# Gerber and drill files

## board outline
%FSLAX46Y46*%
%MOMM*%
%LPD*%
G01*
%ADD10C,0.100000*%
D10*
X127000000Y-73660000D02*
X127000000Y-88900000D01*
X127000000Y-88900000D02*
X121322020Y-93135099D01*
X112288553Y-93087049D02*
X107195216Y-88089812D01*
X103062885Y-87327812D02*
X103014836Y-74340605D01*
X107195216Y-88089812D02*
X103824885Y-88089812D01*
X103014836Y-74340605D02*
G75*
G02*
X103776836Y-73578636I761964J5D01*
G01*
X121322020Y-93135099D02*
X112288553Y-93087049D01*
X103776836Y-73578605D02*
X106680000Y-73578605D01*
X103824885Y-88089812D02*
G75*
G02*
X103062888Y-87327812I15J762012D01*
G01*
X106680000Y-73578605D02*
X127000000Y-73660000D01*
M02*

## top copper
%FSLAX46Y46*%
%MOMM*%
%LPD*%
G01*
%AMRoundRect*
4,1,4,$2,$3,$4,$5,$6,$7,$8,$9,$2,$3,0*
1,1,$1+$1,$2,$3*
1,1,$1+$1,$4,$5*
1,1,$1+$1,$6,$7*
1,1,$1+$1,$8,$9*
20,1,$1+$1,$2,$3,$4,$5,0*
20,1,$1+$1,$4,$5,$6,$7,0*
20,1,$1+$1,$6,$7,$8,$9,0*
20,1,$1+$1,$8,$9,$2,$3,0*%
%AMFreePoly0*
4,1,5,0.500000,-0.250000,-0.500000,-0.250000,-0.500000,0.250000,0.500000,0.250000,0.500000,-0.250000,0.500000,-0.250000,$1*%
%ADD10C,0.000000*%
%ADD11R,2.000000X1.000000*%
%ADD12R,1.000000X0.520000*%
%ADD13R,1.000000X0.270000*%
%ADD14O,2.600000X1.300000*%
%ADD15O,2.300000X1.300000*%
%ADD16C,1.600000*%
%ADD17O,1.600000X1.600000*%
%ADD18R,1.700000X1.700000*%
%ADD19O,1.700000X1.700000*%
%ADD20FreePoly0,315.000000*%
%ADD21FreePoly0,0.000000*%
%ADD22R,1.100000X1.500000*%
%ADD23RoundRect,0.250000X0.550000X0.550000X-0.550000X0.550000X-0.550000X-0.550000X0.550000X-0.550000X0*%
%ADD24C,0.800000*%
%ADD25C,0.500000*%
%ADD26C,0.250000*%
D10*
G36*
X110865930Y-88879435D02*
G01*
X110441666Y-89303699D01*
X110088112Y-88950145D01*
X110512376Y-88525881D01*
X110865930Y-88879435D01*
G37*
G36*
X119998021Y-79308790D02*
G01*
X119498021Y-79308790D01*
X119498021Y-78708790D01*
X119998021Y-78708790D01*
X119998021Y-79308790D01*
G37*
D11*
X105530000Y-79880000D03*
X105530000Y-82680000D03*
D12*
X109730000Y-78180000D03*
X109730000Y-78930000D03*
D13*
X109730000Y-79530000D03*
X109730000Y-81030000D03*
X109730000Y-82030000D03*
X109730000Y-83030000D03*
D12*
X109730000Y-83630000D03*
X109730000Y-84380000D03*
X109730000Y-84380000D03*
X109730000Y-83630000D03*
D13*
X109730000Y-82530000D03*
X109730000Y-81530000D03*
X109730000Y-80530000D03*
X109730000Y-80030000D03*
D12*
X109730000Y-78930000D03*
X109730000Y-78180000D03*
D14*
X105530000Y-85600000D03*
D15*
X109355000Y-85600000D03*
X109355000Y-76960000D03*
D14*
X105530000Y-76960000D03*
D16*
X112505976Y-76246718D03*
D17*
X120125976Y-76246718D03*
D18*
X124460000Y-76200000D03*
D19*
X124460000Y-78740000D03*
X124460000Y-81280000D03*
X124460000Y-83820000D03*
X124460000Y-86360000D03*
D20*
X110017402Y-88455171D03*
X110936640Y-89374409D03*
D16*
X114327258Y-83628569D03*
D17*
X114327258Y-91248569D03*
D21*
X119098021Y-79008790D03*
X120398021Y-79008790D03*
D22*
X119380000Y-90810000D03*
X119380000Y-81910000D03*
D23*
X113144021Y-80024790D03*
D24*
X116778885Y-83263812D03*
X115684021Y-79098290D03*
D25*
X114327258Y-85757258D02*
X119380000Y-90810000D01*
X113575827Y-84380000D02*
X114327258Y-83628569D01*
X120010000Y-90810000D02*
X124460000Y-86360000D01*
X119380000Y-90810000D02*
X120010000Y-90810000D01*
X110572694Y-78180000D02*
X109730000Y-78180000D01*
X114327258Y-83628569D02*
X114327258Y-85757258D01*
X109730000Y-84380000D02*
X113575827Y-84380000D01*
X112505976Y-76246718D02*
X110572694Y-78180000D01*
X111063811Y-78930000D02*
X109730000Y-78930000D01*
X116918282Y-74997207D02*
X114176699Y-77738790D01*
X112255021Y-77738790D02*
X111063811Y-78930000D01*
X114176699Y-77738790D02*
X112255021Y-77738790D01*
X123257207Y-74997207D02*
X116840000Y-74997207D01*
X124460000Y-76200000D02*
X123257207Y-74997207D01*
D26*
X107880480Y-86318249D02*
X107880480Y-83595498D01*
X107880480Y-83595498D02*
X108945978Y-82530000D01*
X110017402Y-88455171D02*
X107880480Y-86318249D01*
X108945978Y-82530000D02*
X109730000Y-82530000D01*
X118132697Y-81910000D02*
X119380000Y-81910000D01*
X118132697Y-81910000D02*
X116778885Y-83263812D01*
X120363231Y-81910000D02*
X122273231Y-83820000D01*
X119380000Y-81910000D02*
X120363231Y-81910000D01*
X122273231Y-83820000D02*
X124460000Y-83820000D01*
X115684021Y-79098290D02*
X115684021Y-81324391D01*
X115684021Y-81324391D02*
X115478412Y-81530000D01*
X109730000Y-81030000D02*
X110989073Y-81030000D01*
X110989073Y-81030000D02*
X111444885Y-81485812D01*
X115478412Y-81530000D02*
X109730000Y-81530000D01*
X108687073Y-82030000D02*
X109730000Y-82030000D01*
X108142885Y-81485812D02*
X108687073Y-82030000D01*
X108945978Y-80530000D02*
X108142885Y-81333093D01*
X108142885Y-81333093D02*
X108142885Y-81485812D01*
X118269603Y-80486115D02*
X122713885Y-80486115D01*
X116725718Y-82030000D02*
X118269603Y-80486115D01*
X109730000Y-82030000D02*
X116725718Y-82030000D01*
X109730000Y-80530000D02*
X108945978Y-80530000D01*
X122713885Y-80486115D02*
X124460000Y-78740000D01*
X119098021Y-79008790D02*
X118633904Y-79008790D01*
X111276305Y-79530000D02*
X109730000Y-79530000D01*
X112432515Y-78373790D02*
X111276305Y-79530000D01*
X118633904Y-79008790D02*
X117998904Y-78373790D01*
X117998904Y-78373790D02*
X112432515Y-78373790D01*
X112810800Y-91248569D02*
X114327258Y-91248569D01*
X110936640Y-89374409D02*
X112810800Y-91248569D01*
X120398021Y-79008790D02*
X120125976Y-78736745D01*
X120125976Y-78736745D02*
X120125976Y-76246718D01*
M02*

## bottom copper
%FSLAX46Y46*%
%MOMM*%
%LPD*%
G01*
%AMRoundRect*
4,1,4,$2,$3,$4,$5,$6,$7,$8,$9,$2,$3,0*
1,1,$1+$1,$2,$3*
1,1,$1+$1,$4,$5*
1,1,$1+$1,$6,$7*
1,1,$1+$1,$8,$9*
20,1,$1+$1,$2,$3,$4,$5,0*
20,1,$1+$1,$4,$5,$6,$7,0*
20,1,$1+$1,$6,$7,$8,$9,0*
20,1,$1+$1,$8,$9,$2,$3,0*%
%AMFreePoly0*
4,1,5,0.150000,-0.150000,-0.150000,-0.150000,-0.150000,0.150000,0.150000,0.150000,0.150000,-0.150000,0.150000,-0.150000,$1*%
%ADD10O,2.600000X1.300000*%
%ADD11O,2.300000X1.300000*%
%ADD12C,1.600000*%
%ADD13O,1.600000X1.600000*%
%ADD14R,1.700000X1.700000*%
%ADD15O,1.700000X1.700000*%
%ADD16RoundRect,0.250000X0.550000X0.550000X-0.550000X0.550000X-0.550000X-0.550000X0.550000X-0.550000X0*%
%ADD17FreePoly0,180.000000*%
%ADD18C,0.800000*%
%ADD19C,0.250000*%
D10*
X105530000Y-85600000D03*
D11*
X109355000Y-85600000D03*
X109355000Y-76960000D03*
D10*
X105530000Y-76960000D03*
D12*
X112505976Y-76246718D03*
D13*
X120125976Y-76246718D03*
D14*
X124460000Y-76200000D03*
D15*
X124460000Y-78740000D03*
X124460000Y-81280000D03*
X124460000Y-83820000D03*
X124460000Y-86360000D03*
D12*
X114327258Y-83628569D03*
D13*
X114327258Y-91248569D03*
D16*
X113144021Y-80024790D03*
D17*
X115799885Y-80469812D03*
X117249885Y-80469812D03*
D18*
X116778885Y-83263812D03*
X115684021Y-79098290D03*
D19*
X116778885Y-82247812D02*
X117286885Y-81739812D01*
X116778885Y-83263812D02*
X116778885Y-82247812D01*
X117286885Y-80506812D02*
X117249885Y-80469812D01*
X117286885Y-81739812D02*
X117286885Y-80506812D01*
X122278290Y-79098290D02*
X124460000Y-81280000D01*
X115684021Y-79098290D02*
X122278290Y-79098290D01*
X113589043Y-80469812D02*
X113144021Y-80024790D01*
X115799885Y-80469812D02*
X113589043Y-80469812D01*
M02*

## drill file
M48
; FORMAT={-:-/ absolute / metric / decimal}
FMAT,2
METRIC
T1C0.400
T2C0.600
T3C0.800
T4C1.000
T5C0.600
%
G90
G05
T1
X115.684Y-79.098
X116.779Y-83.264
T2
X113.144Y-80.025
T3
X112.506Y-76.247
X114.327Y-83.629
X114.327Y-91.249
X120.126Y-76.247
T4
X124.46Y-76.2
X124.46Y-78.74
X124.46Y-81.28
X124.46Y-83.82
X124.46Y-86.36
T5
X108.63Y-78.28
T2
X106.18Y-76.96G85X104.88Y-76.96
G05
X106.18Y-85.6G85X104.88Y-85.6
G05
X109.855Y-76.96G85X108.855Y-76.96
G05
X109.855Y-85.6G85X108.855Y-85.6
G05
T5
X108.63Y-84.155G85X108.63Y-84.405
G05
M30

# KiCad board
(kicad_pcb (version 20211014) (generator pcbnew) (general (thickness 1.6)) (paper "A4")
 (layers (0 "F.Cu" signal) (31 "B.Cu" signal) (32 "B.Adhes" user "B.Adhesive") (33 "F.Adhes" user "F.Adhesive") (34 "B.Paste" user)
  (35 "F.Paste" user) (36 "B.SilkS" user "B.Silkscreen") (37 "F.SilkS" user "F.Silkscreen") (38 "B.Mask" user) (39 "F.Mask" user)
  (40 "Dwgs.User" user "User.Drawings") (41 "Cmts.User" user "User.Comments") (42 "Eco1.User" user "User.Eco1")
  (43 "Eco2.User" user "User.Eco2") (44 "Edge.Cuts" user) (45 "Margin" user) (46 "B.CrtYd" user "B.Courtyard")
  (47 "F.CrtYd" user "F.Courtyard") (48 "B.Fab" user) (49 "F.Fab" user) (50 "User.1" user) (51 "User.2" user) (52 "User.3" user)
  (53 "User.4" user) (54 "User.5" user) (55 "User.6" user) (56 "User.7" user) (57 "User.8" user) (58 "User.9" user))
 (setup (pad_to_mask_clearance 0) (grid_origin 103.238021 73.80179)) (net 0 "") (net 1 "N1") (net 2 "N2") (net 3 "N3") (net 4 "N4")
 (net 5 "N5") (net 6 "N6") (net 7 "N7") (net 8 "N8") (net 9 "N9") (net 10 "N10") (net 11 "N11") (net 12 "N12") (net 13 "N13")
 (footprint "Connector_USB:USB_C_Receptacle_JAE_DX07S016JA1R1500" (layer "F.Cu") (at 106.68 81.28 -90)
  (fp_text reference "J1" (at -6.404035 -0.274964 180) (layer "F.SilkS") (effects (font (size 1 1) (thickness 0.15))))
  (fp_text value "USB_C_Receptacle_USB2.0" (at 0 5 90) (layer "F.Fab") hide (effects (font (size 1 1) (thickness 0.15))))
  (pad "" smd rect (at -1.4 1.15 270) (size 1 2) (layers "F.Cu" "F.Paste" "F.Mask"))
  (pad "" np_thru_hole circle (at -3 -1.95 270) (size 0.6 0.6) (drill 0.6) (layers F&B.Cu *.Mask))
  (pad "" np_thru_hole oval (at 3 -1.95 270) (size 0.85 0.6) (drill oval 0.85 0.6) (layers F&B.Cu *.Mask))
  (pad "" smd rect (at 1.4 1.15 270) (size 1 2) (layers "F.Cu" "F.Paste" "F.Mask"))
  (pad "A1" smd rect (at -3.1 -3.05 270) (size 0.52 1) (layers "F.Cu" "F.Paste" "F.Mask") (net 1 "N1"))
  (pad "A4" smd rect (at -2.35 -3.05 270) (size 0.52 1) (layers "F.Cu" "F.Paste" "F.Mask") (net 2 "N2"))
  (pad "A5" smd rect (at -1.75 -3.05 270) (size 0.27 1) (layers "F.Cu" "F.Paste" "F.Mask") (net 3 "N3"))
  (pad "A6" smd rect (at -0.25 -3.05 270) (size 0.27 1) (layers "F.Cu" "F.Paste" "F.Mask") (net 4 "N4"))
  (pad "A7" smd rect (at 0.75 -3.05 270) (size 0.27 1) (layers "F.Cu" "F.Paste" "F.Mask") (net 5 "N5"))
  (pad "A8" smd rect (at 1.75 -3.05 270) (size 0.27 1) (layers "F.Cu" "F.Paste" "F.Mask") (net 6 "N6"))
  (pad "A9" smd rect (at 2.35 -3.05 270) (size 0.52 1) (layers "F.Cu" "F.Paste" "F.Mask") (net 2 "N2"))
  (pad "A12" smd rect (at 3.1 -3.05 270) (size 0.52 1) (layers "F.Cu" "F.Paste" "F.Mask") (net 1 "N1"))
  (pad "B1" smd rect (at 3.1 -3.05 270) (size 0.52 1) (layers "F.Cu" "F.Paste" "F.Mask") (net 1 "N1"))
  (pad "B4" smd rect (at 2.35 -3.05 270) (size 0.52 1) (layers "F.Cu" "F.Paste" "F.Mask") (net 2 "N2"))
  (pad "B5" smd rect (at 1.25 -3.05 270) (size 0.27 1) (layers "F.Cu" "F.Paste" "F.Mask") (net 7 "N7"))
  (pad "B6" smd rect (at 0.25 -3.05 270) (size 0.27 1) (layers "F.Cu" "F.Paste" "F.Mask") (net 4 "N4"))
  (pad "B7" smd rect (at -0.75 -3.05 270) (size 0.27 1) (layers "F.Cu" "F.Paste" "F.Mask") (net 5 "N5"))
  (pad "B8" smd rect (at -1.25 -3.05 270) (size 0.27 1) (layers "F.Cu" "F.Paste" "F.Mask") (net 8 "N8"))
  (pad "B9" smd rect (at -2.35 -3.05 270) (size 0.52 1) (layers "F.Cu" "F.Paste" "F.Mask") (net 2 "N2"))
  (pad "B12" smd rect (at -3.1 -3.05 270) (size 0.52 1) (layers "F.Cu" "F.Paste" "F.Mask") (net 1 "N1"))
  (pad "S1" thru_hole oval (at 4.32 1.15 270) (size 1.3 2.6) (drill oval 0.6 1.9) (layers *.Cu *.Mask) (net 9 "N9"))
  (pad "S1" thru_hole oval (at 4.32 -2.675 270) (size 1.3 2.3) (drill oval 0.6 1.6) (layers *.Cu *.Mask) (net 9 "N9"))
  (pad "S1" thru_hole oval (at -4.32 -2.675 270) (size 1.3 2.3) (drill oval 0.6 1.6) (layers *.Cu *.Mask) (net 9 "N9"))
  (pad "S1" thru_hole oval (at -4.32 1.15 270) (size 1.3 2.6) (drill oval 0.6 1.9) (layers *.Cu *.Mask) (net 9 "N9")))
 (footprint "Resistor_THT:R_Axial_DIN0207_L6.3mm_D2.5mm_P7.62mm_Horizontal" (layer "F.Cu") (at 112.505976 76.246718)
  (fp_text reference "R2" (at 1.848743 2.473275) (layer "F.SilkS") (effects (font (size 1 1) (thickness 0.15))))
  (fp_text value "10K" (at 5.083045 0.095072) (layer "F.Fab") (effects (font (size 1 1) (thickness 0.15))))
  (pad "1" thru_hole circle (at 0 0) (size 1.6 1.6) (drill 0.8) (layers *.Cu *.Mask) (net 1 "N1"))
  (pad "2" thru_hole oval (at 7.62 0) (size 1.6 1.6) (drill 0.8) (layers *.Cu *.Mask) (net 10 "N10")))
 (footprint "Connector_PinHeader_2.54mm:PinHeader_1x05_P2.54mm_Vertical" (layer "F.Cu") (at 124.46 76.2)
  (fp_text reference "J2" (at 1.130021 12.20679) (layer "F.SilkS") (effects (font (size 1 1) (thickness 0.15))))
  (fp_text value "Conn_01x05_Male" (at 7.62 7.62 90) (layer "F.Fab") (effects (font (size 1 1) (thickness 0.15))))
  (pad "1" thru_hole rect (at 0 0) (size 1.7 1.7) (drill 1) (layers *.Cu *.Mask) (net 2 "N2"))
  (pad "2" thru_hole oval (at 0 2.54) (size 1.7 1.7) (drill 1) (layers *.Cu *.Mask) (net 5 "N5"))
  (pad "3" thru_hole oval (at 0 5.08) (size 1.7 1.7) (drill 1) (layers *.Cu *.Mask) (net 4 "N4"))
  (pad "4" thru_hole oval (at 0 7.62) (size 1.7 1.7) (drill 1) (layers *.Cu *.Mask) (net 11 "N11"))
  (pad "5" thru_hole oval (at 0 10.16) (size 1.7 1.7) (drill 1) (layers *.Cu *.Mask) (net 1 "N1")))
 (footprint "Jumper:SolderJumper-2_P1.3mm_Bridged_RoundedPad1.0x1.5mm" (layer "F.Cu") (at 110.477021 88.91479 -45)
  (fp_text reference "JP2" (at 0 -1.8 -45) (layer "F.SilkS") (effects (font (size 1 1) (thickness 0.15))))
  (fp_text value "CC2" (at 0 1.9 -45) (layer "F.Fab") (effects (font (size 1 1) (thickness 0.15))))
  (fp_poly (pts (xy 0.25 -0.3) (xy -0.25 -0.3) (xy -0.25 0.3) (xy 0.25 0.3)) (layer "F.Cu") (width 0) (fill solid))
  (pad "1" smd custom (at -0.65 0 315) (size 1 0.5) (layers "F.Cu" "F.Mask") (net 7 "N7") (zone_connect 2)
   (options (clearance outline) (anchor rect)) (primitives))
  (pad "2" smd custom (at 0.65 0 315) (size 1 0.5) (layers "F.Cu" "F.Mask") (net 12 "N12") (zone_connect 2)
   (options (clearance outline) (anchor rect)) (primitives)))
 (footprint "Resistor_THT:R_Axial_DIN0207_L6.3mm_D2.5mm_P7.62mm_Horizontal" (layer "F.Cu") (at 114.327258 83.628569 -90)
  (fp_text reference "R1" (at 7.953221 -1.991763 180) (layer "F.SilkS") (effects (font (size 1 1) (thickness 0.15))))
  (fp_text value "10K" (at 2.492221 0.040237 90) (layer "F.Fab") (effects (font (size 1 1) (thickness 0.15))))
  (pad "1" thru_hole circle (at 0 0 270) (size 1.6 1.6) (drill 0.8) (layers *.Cu *.Mask) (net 1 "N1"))
  (pad "2" thru_hole oval (at 7.62 0 270) (size 1.6 1.6) (drill 0.8) (layers *.Cu *.Mask) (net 12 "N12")))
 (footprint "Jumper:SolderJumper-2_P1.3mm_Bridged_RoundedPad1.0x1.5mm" (layer "F.Cu") (at 119.748021 79.00879)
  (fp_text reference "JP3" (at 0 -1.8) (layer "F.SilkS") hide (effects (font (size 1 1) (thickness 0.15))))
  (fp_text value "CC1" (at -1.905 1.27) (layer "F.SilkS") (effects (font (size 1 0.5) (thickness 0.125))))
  (fp_poly (pts (xy 0.25 -0.3) (xy -0.25 -0.3) (xy -0.25 0.3) (xy 0.25 0.3)) (layer "F.Cu") (width 0) (fill solid))
  (pad "1" smd custom (at -0.65 0) (size 1 0.5) (layers "F.Cu" "F.Mask") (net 3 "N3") (zone_connect 2)
   (options (clearance outline) (anchor rect)) (primitives))
  (pad "2" smd custom (at 0.65 0) (size 1 0.5) (layers "F.Cu" "F.Mask") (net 10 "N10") (zone_connect 2)
   (options (clearance outline) (anchor rect)) (primitives)))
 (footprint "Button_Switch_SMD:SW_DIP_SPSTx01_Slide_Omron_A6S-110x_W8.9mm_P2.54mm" (layer "F.Cu") (at 119.38 86.36 90)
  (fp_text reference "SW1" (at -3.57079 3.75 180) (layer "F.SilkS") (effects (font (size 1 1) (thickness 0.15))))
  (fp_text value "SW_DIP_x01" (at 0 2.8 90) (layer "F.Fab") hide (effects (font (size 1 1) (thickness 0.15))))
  (pad "1" smd rect (at -4.45 0 90) (size 1.5 1.1) (layers "F.Cu" "F.Paste" "F.Mask") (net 1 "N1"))
  (pad "2" smd rect (at 4.45 0 90) (size 1.5 1.1) (layers "F.Cu" "F.Paste" "F.Mask") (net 11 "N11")))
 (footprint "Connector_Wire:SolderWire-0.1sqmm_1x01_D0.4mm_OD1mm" (layer "B.Cu") (at 113.144021 80.02479 180)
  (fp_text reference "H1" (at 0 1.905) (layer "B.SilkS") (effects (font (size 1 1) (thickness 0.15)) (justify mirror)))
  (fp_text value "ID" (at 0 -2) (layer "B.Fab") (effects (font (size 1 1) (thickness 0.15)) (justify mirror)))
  (pad "1" thru_hole roundrect (at 0 0 180) (size 1.6 1.6) (drill 0.6) (layers *.Cu *.Mask) (roundrect_rratio 0.15625) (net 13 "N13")))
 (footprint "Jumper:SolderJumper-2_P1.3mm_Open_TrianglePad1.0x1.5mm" (layer "B.Cu") (at 116.524885 80.469812 180)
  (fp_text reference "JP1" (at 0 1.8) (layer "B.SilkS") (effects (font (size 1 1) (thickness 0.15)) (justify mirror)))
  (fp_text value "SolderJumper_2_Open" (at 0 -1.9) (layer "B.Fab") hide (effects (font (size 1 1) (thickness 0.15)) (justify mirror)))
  (pad "1" smd custom (at 0.725 0 180) (size 0.3 0.3) (layers "B.Cu" "B.Mask") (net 13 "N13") (zone_connect 2)
   (options (clearance outline) (anchor rect)) (primitives))
  (pad "2" smd custom (at -0.725 0 180) (size 0.3 0.3) (layers "B.Cu" "B.Mask") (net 11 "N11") (zone_connect 2)
   (options (clearance outline) (anchor rect)) (primitives)))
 (gr_line (start 127 73.66) (end 127 88.9) (layer "Edge.Cuts") (width 0.1))
 (gr_line (start 127 88.9) (end 121.32202 93.135099) (layer "Edge.Cuts") (width 0.1))
 (gr_line (start 112.288553 93.087049) (end 107.195216 88.089812) (layer "Edge.Cuts") (width 0.1))
 (gr_line (start 103.062885 87.327812) (end 103.014836 74.340605) (layer "Edge.Cuts") (width 0.1))
 (gr_line (start 107.195216 88.089812) (end 103.824885 88.089812) (layer "Edge.Cuts") (width 0.1))
 (gr_arc (start 103.014836 74.340605) (mid 103.238021 73.80179) (end 103.776836 73.578605) (layer "Edge.Cuts") (width 0.1))
 (gr_line (start 121.32202 93.135099) (end 112.288553 93.087049) (layer "Edge.Cuts") (width 0.1))
 (gr_line (start 103.776836 73.578605) (end 106.68 73.578605) (layer "Edge.Cuts") (width 0.1))
 (gr_arc (start 103.824885 88.089812) (mid 103.28607 87.866627) (end 103.062885 87.327812) (layer "Edge.Cuts") (width 0.1))
 (gr_line (start 106.68 73.578605) (end 127 73.66) (layer "Edge.Cuts") (width 0.1))
 (segment (start 114.327258 85.757258) (end 119.38 90.81) (width 0.5) (layer "F.Cu") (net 1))
 (segment (start 113.575827 84.38) (end 114.327258 83.628569) (width 0.5) (layer "F.Cu") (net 1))
 (segment (start 120.01 90.81) (end 124.46 86.36) (width 0.5) (layer "F.Cu") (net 1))
 (segment (start 119.38 90.81) (end 120.01 90.81) (width 0.5) (layer "F.Cu") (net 1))
 (segment (start 110.572694 78.18) (end 109.73 78.18) (width 0.5) (layer "F.Cu") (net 1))
 (segment (start 114.327258 83.628569) (end 114.327258 85.757258) (width 0.5) (layer "F.Cu") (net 1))
 (segment (start 109.73 84.38) (end 113.575827 84.38) (width 0.5) (layer "F.Cu") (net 1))
 (segment (start 112.505976 76.246718) (end 110.572694 78.18) (width 0.5) (layer "F.Cu") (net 1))
 (segment (start 111.063811 78.93) (end 109.73 78.93) (width 0.5) (layer "F.Cu") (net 2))
 (segment (start 116.918282 74.997207) (end 114.176699 77.73879) (width 0.5) (layer "F.Cu") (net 2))
 (segment (start 112.255021 77.73879) (end 111.063811 78.93) (width 0.5) (layer "F.Cu") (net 2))
 (segment (start 114.176699 77.73879) (end 112.255021 77.73879) (width 0.5) (layer "F.Cu") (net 2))
 (segment (start 123.257207 74.997207) (end 116.84 74.997207) (width 0.5) (layer "F.Cu") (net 2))
 (segment (start 124.46 76.2) (end 123.257207 74.997207) (width 0.5) (layer "F.Cu") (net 2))
 (segment (start 107.88048 86.318249) (end 107.88048 83.595498) (width 0.25) (layer "F.Cu") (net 7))
 (segment (start 107.88048 83.595498) (end 108.945978 82.53) (width 0.25) (layer "F.Cu") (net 7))
 (segment (start 110.017402 88.455171) (end 107.88048 86.318249) (width 0.25) (layer "F.Cu") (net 7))
 (segment (start 108.945978 82.53) (end 109.73 82.53) (width 0.25) (layer "F.Cu") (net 7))
 (segment (start 118.132697 81.91) (end 119.38 81.91) (width 0.25) (layer "F.Cu") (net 11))
 (segment (start 118.132697 81.91) (end 116.778885 83.263812) (width 0.25) (layer "F.Cu") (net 11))
 (segment (start 120.363231 81.91) (end 122.273231 83.82) (width 0.25) (layer "F.Cu") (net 11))
 (segment (start 119.38 81.91) (end 120.363231 81.91) (width 0.25) (layer "F.Cu") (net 11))
 (segment (start 122.273231 83.82) (end 124.46 83.82) (width 0.25) (layer "F.Cu") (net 11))
 (via (at 116.778885 83.263812) (size 0.8) (drill 0.4) (layers "F.Cu" "B.Cu") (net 11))
 (segment (start 116.778885 82.247812) (end 117.286885 81.739812) (width 0.25) (layer "B.Cu") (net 11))
 (segment (start 116.778885 83.263812) (end 116.778885 82.247812) (width 0.25) (layer "B.Cu") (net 11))
 (segment (start 117.286885 80.506812) (end 117.249885 80.469812) (width 0.25) (layer "B.Cu") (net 11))
 (segment (start 117.286885 81.739812) (end 117.286885 80.506812) (width 0.25) (layer "B.Cu") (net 11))
 (segment (start 115.684021 79.09829) (end 115.684021 81.324391) (width 0.25) (layer "F.Cu") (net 4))
 (segment (start 115.684021 81.324391) (end 115.478412 81.53) (width 0.25) (layer "F.Cu") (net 4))
 (segment (start 109.73 81.03) (end 110.989073 81.03) (width 0.25) (layer "F.Cu") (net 4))
 (segment (start 110.989073 81.03) (end 111.444885 81.485812) (width 0.25) (layer "F.Cu") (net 4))
 (segment (start 115.478412 81.53) (end 109.73 81.53) (width 0.25) (layer "F.Cu") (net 4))
 (via (at 115.684021 79.09829) (size 0.8) (drill 0.4) (layers "F.Cu" "B.Cu") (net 4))
 (segment (start 122.27829 79.09829) (end 124.46 81.28) (width 0.25) (layer "B.Cu") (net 4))
 (segment (start 115.684021 79.09829) (end 122.27829 79.09829) (width 0.25) (layer "B.Cu") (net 4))
 (segment (start 108.687073 82.03) (end 109.73 82.03) (width 0.25) (layer "F.Cu") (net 5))
 (segment (start 108.142885 81.485812) (end 108.687073 82.03) (width 0.25) (layer "F.Cu") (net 5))
 (segment (start 108.945978 80.53) (end 108.142885 81.333093) (width 0.25) (layer "F.Cu") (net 5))
 (segment (start 108.142885 81.333093) (end 108.142885 81.485812) (width 0.25) (layer "F.Cu") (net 5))
 (segment (start 118.269603 80.486115) (end 122.713885 80.486115) (width 0.25) (layer "F.Cu") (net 5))
 (segment (start 116.725718 82.03) (end 118.269603 80.486115) (width 0.25) (layer "F.Cu") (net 5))
 (segment (start 109.73 82.03) (end 116.725718 82.03) (width 0.25) (layer "F.Cu") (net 5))
 (segment (start 109.73 80.53) (end 108.945978 80.53) (width 0.25) (layer "F.Cu") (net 5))
 (segment (start 122.713885 80.486115) (end 124.46 78.74) (width 0.25) (layer "F.Cu") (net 5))
 (segment (start 119.098021 79.00879) (end 118.633904 79.00879) (width 0.25) (layer "F.Cu") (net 3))
 (segment (start 111.276305 79.53) (end 109.73 79.53) (width 0.25) (layer "F.Cu") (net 3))
 (segment (start 112.432515 78.37379) (end 111.276305 79.53) (width 0.25) (layer "F.Cu") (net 3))
 (segment (start 118.633904 79.00879) (end 117.998904 78.37379) (width 0.25) (layer "F.Cu") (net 3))
 (segment (start 117.998904 78.37379) (end 112.432515 78.37379) (width 0.25) (layer "F.Cu") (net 3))
 (segment (start 113.589043 80.469812) (end 113.144021 80.02479) (width 0.25) (layer "B.Cu") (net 13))
 (segment (start 115.799885 80.469812) (end 113.589043 80.469812) (width 0.25) (layer "B.Cu") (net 13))
 (segment (start 112.8108 91.248569) (end 114.327258 91.248569) (width 0.25) (layer "F.Cu") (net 12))
 (segment (start 110.93664 89.374409) (end 112.8108 91.248569) (width 0.25) (layer "F.Cu") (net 12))
 (segment (start 120.398021 79.00879) (end 120.125976 78.736745) (width 0.25) (layer "F.Cu") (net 10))
 (segment (start 120.125976 78.736745) (end 120.125976 76.246718) (width 0.25) (layer "F.Cu") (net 10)))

